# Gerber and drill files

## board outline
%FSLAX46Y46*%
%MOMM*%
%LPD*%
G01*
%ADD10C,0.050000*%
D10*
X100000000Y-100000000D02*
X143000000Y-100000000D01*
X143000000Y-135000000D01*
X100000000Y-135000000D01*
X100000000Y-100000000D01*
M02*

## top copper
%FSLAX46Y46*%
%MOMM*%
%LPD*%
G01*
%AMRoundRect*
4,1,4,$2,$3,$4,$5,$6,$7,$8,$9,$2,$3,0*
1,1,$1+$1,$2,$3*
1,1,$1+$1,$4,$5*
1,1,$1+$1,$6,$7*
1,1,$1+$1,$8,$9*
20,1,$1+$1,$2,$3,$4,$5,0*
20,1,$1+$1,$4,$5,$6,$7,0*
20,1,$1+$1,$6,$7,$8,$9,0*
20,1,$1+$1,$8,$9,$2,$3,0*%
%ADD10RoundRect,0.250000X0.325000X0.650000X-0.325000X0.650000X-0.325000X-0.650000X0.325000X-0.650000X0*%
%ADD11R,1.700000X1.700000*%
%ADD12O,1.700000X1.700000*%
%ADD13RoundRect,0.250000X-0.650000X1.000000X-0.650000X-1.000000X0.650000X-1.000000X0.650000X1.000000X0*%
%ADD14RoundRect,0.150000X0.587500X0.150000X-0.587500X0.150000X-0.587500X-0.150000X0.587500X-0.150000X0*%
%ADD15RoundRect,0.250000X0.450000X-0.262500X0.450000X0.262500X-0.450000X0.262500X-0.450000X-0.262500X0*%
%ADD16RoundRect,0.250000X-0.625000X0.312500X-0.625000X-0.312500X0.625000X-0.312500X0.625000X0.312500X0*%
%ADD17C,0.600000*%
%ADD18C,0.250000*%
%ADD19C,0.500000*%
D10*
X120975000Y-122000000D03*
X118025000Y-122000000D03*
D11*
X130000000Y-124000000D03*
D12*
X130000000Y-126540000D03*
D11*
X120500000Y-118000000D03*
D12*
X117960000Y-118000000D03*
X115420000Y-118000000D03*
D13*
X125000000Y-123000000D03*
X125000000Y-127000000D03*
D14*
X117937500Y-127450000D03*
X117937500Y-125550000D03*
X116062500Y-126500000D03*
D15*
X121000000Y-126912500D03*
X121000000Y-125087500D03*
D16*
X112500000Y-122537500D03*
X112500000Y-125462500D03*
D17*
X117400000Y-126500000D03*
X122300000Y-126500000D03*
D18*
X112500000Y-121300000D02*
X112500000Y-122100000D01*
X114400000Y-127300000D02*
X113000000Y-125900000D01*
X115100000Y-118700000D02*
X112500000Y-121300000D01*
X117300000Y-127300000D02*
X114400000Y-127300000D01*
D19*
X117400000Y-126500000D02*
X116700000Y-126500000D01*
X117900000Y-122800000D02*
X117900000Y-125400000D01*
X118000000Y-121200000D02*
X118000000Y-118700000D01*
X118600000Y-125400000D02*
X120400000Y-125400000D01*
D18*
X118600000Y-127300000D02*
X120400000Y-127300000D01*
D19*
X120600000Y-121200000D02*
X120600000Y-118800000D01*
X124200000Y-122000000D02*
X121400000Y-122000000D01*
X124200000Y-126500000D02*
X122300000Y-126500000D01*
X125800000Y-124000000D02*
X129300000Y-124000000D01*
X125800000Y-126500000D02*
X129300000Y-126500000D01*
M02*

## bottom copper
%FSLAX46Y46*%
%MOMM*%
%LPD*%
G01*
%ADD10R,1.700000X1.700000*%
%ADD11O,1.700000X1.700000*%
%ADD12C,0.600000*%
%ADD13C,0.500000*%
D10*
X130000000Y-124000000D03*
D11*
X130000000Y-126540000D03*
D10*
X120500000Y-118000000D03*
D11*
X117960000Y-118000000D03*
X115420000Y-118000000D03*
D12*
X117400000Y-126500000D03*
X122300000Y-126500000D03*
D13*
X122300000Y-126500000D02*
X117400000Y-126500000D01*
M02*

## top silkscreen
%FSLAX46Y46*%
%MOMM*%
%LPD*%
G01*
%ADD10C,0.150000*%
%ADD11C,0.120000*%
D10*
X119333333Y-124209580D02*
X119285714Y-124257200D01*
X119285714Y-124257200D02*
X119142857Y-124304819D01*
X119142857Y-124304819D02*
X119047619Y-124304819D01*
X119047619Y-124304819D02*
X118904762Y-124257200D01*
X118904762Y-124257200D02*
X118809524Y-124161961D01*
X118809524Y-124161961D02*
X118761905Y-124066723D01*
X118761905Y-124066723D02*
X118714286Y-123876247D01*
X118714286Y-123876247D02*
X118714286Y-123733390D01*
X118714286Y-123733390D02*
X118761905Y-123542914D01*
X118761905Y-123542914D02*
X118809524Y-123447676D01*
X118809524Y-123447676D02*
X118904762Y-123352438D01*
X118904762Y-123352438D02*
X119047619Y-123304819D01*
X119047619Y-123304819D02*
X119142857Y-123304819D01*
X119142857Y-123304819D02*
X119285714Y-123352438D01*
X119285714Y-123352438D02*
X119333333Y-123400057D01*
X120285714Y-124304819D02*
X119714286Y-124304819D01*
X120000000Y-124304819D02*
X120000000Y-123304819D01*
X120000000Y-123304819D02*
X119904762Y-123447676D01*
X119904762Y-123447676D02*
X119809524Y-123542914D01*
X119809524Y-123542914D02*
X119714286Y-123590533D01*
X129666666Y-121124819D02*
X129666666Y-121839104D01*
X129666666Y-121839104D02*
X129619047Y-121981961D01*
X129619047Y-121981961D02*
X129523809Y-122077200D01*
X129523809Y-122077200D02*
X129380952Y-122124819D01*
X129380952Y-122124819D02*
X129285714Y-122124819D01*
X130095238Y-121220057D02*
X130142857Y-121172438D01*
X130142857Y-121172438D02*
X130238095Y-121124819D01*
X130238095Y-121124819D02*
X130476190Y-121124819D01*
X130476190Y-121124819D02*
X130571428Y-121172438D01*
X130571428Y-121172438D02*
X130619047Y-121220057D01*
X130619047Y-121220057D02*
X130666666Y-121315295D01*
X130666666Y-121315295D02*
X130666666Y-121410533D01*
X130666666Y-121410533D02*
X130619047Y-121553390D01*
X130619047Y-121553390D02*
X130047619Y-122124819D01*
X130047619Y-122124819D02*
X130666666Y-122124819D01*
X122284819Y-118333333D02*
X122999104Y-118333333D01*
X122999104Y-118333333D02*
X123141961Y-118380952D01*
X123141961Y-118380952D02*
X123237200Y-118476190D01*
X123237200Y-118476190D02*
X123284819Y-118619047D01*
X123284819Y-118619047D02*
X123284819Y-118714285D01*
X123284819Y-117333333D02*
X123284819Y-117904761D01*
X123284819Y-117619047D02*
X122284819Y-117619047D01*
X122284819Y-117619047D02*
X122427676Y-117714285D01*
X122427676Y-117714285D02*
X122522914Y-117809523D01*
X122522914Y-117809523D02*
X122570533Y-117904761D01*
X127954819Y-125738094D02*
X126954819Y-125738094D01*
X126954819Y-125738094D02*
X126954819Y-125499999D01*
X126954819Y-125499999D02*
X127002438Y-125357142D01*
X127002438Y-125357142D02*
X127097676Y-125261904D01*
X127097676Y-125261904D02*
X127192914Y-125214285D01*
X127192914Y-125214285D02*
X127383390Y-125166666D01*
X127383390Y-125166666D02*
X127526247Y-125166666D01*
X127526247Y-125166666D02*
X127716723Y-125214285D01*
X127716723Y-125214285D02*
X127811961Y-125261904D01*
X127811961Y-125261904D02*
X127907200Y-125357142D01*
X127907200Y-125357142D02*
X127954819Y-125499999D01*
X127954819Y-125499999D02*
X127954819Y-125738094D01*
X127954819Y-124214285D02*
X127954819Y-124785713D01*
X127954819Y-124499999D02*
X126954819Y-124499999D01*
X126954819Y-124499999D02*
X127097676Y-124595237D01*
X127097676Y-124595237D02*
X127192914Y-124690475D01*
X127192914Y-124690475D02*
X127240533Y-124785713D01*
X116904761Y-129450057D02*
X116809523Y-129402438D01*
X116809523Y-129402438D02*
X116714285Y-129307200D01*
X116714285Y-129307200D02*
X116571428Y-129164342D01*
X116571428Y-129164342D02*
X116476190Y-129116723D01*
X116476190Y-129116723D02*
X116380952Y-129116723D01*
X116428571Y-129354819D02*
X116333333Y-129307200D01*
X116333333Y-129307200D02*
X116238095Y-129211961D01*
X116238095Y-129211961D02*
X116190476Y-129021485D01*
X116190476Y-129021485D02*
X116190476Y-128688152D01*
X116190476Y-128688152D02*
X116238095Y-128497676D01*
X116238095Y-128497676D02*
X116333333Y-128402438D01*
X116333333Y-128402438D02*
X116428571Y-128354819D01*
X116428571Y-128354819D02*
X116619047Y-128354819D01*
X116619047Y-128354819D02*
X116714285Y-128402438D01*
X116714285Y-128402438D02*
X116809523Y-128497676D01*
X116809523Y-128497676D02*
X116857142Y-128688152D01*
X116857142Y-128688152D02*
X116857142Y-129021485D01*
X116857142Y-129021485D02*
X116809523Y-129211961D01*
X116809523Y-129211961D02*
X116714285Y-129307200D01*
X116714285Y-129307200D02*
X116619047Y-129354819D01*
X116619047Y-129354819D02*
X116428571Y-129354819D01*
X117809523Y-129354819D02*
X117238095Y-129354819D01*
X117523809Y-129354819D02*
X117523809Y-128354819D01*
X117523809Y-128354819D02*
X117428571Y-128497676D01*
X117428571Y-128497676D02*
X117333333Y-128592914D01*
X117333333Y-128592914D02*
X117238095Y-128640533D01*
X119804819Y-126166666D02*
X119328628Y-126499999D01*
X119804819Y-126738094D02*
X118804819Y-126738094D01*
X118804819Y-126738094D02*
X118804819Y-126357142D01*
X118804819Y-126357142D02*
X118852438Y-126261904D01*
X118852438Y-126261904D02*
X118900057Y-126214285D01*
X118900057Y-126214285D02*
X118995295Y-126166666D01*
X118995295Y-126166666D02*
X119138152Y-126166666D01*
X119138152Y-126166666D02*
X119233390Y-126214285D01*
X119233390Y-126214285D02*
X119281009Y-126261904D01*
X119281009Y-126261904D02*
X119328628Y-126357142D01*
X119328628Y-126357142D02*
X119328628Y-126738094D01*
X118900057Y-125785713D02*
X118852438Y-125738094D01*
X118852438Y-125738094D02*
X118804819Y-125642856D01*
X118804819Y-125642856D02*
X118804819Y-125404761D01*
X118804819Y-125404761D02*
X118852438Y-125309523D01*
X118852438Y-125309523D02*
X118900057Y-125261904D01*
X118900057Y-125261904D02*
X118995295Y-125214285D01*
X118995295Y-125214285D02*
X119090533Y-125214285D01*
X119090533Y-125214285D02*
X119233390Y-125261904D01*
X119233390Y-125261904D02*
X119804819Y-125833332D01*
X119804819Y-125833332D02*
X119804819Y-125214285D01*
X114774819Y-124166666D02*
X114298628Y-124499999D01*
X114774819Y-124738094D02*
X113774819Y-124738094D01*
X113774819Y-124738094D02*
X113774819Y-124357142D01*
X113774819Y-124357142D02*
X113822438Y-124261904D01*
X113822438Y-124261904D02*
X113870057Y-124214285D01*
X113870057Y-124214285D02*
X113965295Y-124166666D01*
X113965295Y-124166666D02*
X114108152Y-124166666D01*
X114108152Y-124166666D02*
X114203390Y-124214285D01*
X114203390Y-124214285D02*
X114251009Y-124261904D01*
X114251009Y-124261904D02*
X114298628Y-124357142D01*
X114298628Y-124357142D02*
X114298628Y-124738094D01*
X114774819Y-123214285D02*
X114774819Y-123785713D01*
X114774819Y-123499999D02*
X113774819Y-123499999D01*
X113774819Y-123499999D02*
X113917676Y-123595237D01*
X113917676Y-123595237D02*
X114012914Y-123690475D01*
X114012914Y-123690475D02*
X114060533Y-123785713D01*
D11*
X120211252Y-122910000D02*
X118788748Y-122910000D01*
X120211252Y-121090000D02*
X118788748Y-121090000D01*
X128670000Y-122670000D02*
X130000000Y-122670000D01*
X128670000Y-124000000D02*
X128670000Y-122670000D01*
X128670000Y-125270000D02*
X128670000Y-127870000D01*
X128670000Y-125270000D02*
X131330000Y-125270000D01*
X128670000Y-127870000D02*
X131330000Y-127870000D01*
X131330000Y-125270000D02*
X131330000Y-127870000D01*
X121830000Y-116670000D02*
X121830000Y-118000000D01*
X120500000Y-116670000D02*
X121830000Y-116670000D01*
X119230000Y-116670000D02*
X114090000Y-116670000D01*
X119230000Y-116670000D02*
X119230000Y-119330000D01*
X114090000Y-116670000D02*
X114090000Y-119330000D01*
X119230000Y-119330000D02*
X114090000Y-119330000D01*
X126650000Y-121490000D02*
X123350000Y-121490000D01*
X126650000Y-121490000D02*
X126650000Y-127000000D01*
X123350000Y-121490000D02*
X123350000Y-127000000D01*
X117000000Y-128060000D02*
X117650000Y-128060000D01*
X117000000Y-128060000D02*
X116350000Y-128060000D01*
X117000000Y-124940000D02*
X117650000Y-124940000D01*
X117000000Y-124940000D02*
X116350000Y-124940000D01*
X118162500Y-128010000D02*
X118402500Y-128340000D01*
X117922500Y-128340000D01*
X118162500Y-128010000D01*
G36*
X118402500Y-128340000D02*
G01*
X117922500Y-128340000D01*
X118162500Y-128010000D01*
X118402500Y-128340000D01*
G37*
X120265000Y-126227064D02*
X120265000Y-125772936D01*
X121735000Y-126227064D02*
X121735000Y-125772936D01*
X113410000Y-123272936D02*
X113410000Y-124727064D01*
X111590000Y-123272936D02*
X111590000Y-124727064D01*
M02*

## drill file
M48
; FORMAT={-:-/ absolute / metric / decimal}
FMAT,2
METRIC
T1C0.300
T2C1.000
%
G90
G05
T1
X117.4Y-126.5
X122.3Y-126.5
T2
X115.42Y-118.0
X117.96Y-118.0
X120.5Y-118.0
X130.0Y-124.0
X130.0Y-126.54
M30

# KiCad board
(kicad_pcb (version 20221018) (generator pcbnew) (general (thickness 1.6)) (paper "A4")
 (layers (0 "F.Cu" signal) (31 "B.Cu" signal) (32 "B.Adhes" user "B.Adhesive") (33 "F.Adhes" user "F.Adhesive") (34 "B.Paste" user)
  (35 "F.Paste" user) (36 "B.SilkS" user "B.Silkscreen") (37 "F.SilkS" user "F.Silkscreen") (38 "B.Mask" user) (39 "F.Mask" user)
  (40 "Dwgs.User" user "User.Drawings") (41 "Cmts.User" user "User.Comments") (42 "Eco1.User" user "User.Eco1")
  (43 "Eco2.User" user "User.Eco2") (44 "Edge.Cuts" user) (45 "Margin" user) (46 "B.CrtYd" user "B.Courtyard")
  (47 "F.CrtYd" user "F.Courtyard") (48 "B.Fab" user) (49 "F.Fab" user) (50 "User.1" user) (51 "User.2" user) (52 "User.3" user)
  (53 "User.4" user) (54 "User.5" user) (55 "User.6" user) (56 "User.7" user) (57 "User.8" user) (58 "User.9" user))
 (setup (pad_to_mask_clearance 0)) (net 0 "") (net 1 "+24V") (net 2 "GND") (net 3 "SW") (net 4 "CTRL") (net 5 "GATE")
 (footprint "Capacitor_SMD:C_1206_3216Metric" (layer "F.Cu") (at 119.5 122 180)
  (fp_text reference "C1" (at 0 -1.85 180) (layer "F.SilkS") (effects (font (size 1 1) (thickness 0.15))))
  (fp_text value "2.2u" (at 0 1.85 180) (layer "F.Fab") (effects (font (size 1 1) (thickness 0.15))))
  (fp_line (start -0.711252 -0.91) (end 0.711252 -0.91) (stroke (width 0.12) (type solid)) (layer "F.SilkS"))
  (fp_line (start -0.711252 0.91) (end 0.711252 0.91) (stroke (width 0.12) (type solid)) (layer "F.SilkS"))
  (pad "1" smd roundrect (at -1.475 0 180) (size 1.15 1.8) (layers "F.Cu" "F.Paste" "F.Mask") (roundrect_rratio 0.217391) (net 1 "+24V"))
  (pad "2" smd roundrect (at 1.475 0 180) (size 1.15 1.8) (layers "F.Cu" "F.Paste" "F.Mask") (roundrect_rratio 0.217391) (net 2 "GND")))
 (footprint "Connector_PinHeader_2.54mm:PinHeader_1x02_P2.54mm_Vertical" (layer "F.Cu") (at 130 124)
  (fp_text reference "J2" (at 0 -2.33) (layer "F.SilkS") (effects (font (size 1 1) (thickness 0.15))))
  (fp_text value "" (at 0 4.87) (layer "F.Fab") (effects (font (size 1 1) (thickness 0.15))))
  (fp_line (start -1.33 -1.33) (end 0 -1.33) (stroke (width 0.12) (type solid)) (layer "F.SilkS"))
  (fp_line (start -1.33 0) (end -1.33 -1.33) (stroke (width 0.12) (type solid)) (layer "F.SilkS"))
  (fp_line (start -1.33 1.27) (end -1.33 3.87) (stroke (width 0.12) (type solid)) (layer "F.SilkS"))
  (fp_line (start -1.33 1.27) (end 1.33 1.27) (stroke (width 0.12) (type solid)) (layer "F.SilkS"))
  (fp_line (start -1.33 3.87) (end 1.33 3.87) (stroke (width 0.12) (type solid)) (layer "F.SilkS"))
  (fp_line (start 1.33 1.27) (end 1.33 3.87) (stroke (width 0.12) (type solid)) (layer "F.SilkS"))
  (pad "1" thru_hole rect (at 0 0) (size 1.7 1.7) (drill 1) (layers "*.Cu" "*.Mask") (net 1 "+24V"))
  (pad "2" thru_hole oval (at 0 2.54) (size 1.7 1.7) (drill 1) (layers "*.Cu" "*.Mask") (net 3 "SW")))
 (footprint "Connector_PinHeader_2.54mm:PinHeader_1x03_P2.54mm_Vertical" (layer "F.Cu") (at 120.5 118 -90)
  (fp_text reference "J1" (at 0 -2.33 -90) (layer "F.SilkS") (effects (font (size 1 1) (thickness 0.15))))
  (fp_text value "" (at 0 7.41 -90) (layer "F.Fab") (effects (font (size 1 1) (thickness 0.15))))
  (fp_line (start -1.33 -1.33) (end 0 -1.33) (stroke (width 0.12) (type solid)) (layer "F.SilkS"))
  (fp_line (start -1.33 0) (end -1.33 -1.33) (stroke (width 0.12) (type solid)) (layer "F.SilkS"))
  (fp_line (start -1.33 1.27) (end -1.33 6.41) (stroke (width 0.12) (type solid)) (layer "F.SilkS"))
  (fp_line (start -1.33 1.27) (end 1.33 1.27) (stroke (width 0.12) (type solid)) (layer "F.SilkS"))
  (fp_line (start -1.33 6.41) (end 1.33 6.41) (stroke (width 0.12) (type solid)) (layer "F.SilkS"))
  (fp_line (start 1.33 1.27) (end 1.33 6.41) (stroke (width 0.12) (type solid)) (layer "F.SilkS"))
  (pad "1" thru_hole rect (at 0 0 270) (size 1.7 1.7) (drill 1) (layers "*.Cu" "*.Mask") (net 1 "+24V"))
  (pad "2" thru_hole oval (at 0 2.54 270) (size 1.7 1.7) (drill 1) (layers "*.Cu" "*.Mask") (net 2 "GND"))
  (pad "3" thru_hole oval (at 0 5.08 270) (size 1.7 1.7) (drill 1) (layers "*.Cu" "*.Mask") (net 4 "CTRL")))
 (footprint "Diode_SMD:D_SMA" (layer "F.Cu") (at 125 125 -90)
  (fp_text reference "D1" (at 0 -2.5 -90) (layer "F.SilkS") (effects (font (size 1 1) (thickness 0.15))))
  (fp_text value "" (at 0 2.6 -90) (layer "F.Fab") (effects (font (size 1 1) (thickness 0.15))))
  (fp_line (start -3.51 -1.65) (end -3.51 1.65) (stroke (width 0.12) (type solid)) (layer "F.SilkS"))
  (fp_line (start -3.51 -1.65) (end 2 -1.65) (stroke (width 0.12) (type solid)) (layer "F.SilkS"))
  (fp_line (start -3.51 1.65) (end 2 1.65) (stroke (width 0.12) (type solid)) (layer "F.SilkS"))
  (pad "1" smd roundrect (at -2 0 270) (size 2.5 1.8) (layers "F.Cu" "F.Paste" "F.Mask") (roundrect_rratio 0.1388888889) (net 1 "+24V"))
  (pad "2" smd roundrect (at 2 0 270) (size 2.5 1.8) (layers "F.Cu" "F.Paste" "F.Mask") (roundrect_rratio 0.1388888889) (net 3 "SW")))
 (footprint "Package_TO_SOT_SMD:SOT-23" (layer "F.Cu") (at 117 126.5 180)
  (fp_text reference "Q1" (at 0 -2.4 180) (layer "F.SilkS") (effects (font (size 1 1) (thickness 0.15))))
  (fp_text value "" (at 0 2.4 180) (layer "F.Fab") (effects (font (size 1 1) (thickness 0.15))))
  (fp_line (start 0 -1.56) (end -0.65 -1.56) (stroke (width 0.12) (type solid)) (layer "F.SilkS"))
  (fp_line (start 0 -1.56) (end 0.65 -1.56) (stroke (width 0.12) (type solid)) (layer "F.SilkS"))
  (fp_line (start 0 1.56) (end -0.65 1.56) (stroke (width 0.12) (type solid)) (layer "F.SilkS"))
  (fp_line (start 0 1.56) (end 0.65 1.56) (stroke (width 0.12) (type solid)) (layer "F.SilkS"))
  (fp_poly
   (pts (xy -1.1625 -1.51) (xy -1.4025 -1.84) (xy -0.9225 -1.84) (xy -1.1625 -1.51)) (stroke (width 0.12) (type solid)) (fill solid)
   (layer "F.SilkS"))
  (pad "1" smd roundrect (at -0.9375 -0.95 180) (size 1.475 0.6) (layers "F.Cu" "F.Paste" "F.Mask") (roundrect_rratio 0.25) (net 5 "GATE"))
  (pad "2" smd roundrect (at -0.9375 0.95 180) (size 1.475 0.6) (layers "F.Cu" "F.Paste" "F.Mask") (roundrect_rratio 0.25) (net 2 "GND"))
  (pad "3" smd roundrect (at 0.9375 0 180) (size 1.475 0.6) (layers "F.Cu" "F.Paste" "F.Mask") (roundrect_rratio 0.25) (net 3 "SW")))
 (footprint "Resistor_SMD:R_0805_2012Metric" (layer "F.Cu") (at 121 126 90)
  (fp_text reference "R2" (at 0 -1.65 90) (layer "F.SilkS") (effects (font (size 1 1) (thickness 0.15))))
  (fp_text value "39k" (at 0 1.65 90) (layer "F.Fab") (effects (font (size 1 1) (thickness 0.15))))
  (fp_line (start -0.227064 -0.735) (end 0.227064 -0.735) (stroke (width 0.12) (type solid)) (layer "F.SilkS"))
  (fp_line (start -0.227064 0.735) (end 0.227064 0.735) (stroke (width 0.12) (type solid)) (layer "F.SilkS"))
  (pad "1" smd roundrect (at -0.9125 0 90) (size 1.025 1.4) (layers "F.Cu" "F.Paste" "F.Mask") (roundrect_rratio 0.243902) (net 5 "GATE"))
  (pad "2" smd roundrect (at 0.9125 0 90) (size 1.025 1.4) (layers "F.Cu" "F.Paste" "F.Mask") (roundrect_rratio 0.243902) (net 2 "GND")))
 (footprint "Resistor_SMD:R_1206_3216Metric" (layer "F.Cu") (at 112.5 124 -90)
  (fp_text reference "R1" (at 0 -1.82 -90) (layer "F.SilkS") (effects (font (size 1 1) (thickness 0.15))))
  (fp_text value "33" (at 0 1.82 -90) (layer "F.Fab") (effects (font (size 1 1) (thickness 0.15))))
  (fp_line (start -0.727064 -0.91) (end 0.727064 -0.91) (stroke (width 0.12) (type solid)) (layer "F.SilkS"))
  (fp_line (start -0.727064 0.91) (end 0.727064 0.91) (stroke (width 0.12) (type solid)) (layer "F.SilkS"))
  (pad "1" smd roundrect (at -1.4625 0 270) (size 1.125 1.75) (layers "F.Cu" "F.Paste" "F.Mask") (roundrect_rratio 0.222222) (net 4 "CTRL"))
  (pad "2" smd roundrect (at 1.4625 0 270) (size 1.125 1.75) (layers "F.Cu" "F.Paste" "F.Mask") (roundrect_rratio 0.222222) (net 5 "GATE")))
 (gr_rect (start 100 100) (end 143 135) (stroke (width 0.05) (type default)) (fill none) (layer "Edge.Cuts"))
 (segment (start 112.5 121.3) (end 112.5 122.1) (width 0.25) (layer "F.Cu") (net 4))
 (segment (start 114.4 127.3) (end 113 125.9) (width 0.25) (layer "F.Cu") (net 5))
 (segment (start 115.1 118.7) (end 112.5 121.3) (width 0.25) (layer "F.Cu") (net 4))
 (segment (start 117.3 127.3) (end 114.4 127.3) (width 0.25) (layer "F.Cu") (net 5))
 (segment (start 117.4 126.5) (end 116.7 126.5) (width 0.5) (layer "F.Cu") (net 3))
 (segment (start 117.9 122.8) (end 117.9 125.4) (width 0.5) (layer "F.Cu") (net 2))
 (segment (start 118 121.2) (end 118 118.7) (width 0.5) (layer "F.Cu") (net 2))
 (segment (start 118.6 125.4) (end 120.4 125.4) (width 0.5) (layer "F.Cu") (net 2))
 (segment (start 118.6 127.3) (end 120.4 127.3) (width 0.25) (layer "F.Cu") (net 5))
 (segment (start 120.6 121.2) (end 120.6 118.8) (width 0.5) (layer "F.Cu") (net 1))
 (segment (start 124.2 122) (end 121.4 122) (width 0.5) (layer "F.Cu") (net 1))
 (segment (start 124.2 126.5) (end 122.3 126.5) (width 0.5) (layer "F.Cu") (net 3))
 (segment (start 125.8 124) (end 129.3 124) (width 0.5) (layer "F.Cu") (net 1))
 (segment (start 125.8 126.5) (end 129.3 126.5) (width 0.5) (layer "F.Cu") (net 3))
 (via (at 117.4 126.5) (size 0.6) (drill 0.3) (layers "F.Cu" "B.Cu") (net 3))
 (via (at 122.3 126.5) (size 0.6) (drill 0.3) (layers "F.Cu" "B.Cu") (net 3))
 (segment (start 122.3 126.5) (end 117.4 126.5) (width 0.5) (layer "B.Cu") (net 3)))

